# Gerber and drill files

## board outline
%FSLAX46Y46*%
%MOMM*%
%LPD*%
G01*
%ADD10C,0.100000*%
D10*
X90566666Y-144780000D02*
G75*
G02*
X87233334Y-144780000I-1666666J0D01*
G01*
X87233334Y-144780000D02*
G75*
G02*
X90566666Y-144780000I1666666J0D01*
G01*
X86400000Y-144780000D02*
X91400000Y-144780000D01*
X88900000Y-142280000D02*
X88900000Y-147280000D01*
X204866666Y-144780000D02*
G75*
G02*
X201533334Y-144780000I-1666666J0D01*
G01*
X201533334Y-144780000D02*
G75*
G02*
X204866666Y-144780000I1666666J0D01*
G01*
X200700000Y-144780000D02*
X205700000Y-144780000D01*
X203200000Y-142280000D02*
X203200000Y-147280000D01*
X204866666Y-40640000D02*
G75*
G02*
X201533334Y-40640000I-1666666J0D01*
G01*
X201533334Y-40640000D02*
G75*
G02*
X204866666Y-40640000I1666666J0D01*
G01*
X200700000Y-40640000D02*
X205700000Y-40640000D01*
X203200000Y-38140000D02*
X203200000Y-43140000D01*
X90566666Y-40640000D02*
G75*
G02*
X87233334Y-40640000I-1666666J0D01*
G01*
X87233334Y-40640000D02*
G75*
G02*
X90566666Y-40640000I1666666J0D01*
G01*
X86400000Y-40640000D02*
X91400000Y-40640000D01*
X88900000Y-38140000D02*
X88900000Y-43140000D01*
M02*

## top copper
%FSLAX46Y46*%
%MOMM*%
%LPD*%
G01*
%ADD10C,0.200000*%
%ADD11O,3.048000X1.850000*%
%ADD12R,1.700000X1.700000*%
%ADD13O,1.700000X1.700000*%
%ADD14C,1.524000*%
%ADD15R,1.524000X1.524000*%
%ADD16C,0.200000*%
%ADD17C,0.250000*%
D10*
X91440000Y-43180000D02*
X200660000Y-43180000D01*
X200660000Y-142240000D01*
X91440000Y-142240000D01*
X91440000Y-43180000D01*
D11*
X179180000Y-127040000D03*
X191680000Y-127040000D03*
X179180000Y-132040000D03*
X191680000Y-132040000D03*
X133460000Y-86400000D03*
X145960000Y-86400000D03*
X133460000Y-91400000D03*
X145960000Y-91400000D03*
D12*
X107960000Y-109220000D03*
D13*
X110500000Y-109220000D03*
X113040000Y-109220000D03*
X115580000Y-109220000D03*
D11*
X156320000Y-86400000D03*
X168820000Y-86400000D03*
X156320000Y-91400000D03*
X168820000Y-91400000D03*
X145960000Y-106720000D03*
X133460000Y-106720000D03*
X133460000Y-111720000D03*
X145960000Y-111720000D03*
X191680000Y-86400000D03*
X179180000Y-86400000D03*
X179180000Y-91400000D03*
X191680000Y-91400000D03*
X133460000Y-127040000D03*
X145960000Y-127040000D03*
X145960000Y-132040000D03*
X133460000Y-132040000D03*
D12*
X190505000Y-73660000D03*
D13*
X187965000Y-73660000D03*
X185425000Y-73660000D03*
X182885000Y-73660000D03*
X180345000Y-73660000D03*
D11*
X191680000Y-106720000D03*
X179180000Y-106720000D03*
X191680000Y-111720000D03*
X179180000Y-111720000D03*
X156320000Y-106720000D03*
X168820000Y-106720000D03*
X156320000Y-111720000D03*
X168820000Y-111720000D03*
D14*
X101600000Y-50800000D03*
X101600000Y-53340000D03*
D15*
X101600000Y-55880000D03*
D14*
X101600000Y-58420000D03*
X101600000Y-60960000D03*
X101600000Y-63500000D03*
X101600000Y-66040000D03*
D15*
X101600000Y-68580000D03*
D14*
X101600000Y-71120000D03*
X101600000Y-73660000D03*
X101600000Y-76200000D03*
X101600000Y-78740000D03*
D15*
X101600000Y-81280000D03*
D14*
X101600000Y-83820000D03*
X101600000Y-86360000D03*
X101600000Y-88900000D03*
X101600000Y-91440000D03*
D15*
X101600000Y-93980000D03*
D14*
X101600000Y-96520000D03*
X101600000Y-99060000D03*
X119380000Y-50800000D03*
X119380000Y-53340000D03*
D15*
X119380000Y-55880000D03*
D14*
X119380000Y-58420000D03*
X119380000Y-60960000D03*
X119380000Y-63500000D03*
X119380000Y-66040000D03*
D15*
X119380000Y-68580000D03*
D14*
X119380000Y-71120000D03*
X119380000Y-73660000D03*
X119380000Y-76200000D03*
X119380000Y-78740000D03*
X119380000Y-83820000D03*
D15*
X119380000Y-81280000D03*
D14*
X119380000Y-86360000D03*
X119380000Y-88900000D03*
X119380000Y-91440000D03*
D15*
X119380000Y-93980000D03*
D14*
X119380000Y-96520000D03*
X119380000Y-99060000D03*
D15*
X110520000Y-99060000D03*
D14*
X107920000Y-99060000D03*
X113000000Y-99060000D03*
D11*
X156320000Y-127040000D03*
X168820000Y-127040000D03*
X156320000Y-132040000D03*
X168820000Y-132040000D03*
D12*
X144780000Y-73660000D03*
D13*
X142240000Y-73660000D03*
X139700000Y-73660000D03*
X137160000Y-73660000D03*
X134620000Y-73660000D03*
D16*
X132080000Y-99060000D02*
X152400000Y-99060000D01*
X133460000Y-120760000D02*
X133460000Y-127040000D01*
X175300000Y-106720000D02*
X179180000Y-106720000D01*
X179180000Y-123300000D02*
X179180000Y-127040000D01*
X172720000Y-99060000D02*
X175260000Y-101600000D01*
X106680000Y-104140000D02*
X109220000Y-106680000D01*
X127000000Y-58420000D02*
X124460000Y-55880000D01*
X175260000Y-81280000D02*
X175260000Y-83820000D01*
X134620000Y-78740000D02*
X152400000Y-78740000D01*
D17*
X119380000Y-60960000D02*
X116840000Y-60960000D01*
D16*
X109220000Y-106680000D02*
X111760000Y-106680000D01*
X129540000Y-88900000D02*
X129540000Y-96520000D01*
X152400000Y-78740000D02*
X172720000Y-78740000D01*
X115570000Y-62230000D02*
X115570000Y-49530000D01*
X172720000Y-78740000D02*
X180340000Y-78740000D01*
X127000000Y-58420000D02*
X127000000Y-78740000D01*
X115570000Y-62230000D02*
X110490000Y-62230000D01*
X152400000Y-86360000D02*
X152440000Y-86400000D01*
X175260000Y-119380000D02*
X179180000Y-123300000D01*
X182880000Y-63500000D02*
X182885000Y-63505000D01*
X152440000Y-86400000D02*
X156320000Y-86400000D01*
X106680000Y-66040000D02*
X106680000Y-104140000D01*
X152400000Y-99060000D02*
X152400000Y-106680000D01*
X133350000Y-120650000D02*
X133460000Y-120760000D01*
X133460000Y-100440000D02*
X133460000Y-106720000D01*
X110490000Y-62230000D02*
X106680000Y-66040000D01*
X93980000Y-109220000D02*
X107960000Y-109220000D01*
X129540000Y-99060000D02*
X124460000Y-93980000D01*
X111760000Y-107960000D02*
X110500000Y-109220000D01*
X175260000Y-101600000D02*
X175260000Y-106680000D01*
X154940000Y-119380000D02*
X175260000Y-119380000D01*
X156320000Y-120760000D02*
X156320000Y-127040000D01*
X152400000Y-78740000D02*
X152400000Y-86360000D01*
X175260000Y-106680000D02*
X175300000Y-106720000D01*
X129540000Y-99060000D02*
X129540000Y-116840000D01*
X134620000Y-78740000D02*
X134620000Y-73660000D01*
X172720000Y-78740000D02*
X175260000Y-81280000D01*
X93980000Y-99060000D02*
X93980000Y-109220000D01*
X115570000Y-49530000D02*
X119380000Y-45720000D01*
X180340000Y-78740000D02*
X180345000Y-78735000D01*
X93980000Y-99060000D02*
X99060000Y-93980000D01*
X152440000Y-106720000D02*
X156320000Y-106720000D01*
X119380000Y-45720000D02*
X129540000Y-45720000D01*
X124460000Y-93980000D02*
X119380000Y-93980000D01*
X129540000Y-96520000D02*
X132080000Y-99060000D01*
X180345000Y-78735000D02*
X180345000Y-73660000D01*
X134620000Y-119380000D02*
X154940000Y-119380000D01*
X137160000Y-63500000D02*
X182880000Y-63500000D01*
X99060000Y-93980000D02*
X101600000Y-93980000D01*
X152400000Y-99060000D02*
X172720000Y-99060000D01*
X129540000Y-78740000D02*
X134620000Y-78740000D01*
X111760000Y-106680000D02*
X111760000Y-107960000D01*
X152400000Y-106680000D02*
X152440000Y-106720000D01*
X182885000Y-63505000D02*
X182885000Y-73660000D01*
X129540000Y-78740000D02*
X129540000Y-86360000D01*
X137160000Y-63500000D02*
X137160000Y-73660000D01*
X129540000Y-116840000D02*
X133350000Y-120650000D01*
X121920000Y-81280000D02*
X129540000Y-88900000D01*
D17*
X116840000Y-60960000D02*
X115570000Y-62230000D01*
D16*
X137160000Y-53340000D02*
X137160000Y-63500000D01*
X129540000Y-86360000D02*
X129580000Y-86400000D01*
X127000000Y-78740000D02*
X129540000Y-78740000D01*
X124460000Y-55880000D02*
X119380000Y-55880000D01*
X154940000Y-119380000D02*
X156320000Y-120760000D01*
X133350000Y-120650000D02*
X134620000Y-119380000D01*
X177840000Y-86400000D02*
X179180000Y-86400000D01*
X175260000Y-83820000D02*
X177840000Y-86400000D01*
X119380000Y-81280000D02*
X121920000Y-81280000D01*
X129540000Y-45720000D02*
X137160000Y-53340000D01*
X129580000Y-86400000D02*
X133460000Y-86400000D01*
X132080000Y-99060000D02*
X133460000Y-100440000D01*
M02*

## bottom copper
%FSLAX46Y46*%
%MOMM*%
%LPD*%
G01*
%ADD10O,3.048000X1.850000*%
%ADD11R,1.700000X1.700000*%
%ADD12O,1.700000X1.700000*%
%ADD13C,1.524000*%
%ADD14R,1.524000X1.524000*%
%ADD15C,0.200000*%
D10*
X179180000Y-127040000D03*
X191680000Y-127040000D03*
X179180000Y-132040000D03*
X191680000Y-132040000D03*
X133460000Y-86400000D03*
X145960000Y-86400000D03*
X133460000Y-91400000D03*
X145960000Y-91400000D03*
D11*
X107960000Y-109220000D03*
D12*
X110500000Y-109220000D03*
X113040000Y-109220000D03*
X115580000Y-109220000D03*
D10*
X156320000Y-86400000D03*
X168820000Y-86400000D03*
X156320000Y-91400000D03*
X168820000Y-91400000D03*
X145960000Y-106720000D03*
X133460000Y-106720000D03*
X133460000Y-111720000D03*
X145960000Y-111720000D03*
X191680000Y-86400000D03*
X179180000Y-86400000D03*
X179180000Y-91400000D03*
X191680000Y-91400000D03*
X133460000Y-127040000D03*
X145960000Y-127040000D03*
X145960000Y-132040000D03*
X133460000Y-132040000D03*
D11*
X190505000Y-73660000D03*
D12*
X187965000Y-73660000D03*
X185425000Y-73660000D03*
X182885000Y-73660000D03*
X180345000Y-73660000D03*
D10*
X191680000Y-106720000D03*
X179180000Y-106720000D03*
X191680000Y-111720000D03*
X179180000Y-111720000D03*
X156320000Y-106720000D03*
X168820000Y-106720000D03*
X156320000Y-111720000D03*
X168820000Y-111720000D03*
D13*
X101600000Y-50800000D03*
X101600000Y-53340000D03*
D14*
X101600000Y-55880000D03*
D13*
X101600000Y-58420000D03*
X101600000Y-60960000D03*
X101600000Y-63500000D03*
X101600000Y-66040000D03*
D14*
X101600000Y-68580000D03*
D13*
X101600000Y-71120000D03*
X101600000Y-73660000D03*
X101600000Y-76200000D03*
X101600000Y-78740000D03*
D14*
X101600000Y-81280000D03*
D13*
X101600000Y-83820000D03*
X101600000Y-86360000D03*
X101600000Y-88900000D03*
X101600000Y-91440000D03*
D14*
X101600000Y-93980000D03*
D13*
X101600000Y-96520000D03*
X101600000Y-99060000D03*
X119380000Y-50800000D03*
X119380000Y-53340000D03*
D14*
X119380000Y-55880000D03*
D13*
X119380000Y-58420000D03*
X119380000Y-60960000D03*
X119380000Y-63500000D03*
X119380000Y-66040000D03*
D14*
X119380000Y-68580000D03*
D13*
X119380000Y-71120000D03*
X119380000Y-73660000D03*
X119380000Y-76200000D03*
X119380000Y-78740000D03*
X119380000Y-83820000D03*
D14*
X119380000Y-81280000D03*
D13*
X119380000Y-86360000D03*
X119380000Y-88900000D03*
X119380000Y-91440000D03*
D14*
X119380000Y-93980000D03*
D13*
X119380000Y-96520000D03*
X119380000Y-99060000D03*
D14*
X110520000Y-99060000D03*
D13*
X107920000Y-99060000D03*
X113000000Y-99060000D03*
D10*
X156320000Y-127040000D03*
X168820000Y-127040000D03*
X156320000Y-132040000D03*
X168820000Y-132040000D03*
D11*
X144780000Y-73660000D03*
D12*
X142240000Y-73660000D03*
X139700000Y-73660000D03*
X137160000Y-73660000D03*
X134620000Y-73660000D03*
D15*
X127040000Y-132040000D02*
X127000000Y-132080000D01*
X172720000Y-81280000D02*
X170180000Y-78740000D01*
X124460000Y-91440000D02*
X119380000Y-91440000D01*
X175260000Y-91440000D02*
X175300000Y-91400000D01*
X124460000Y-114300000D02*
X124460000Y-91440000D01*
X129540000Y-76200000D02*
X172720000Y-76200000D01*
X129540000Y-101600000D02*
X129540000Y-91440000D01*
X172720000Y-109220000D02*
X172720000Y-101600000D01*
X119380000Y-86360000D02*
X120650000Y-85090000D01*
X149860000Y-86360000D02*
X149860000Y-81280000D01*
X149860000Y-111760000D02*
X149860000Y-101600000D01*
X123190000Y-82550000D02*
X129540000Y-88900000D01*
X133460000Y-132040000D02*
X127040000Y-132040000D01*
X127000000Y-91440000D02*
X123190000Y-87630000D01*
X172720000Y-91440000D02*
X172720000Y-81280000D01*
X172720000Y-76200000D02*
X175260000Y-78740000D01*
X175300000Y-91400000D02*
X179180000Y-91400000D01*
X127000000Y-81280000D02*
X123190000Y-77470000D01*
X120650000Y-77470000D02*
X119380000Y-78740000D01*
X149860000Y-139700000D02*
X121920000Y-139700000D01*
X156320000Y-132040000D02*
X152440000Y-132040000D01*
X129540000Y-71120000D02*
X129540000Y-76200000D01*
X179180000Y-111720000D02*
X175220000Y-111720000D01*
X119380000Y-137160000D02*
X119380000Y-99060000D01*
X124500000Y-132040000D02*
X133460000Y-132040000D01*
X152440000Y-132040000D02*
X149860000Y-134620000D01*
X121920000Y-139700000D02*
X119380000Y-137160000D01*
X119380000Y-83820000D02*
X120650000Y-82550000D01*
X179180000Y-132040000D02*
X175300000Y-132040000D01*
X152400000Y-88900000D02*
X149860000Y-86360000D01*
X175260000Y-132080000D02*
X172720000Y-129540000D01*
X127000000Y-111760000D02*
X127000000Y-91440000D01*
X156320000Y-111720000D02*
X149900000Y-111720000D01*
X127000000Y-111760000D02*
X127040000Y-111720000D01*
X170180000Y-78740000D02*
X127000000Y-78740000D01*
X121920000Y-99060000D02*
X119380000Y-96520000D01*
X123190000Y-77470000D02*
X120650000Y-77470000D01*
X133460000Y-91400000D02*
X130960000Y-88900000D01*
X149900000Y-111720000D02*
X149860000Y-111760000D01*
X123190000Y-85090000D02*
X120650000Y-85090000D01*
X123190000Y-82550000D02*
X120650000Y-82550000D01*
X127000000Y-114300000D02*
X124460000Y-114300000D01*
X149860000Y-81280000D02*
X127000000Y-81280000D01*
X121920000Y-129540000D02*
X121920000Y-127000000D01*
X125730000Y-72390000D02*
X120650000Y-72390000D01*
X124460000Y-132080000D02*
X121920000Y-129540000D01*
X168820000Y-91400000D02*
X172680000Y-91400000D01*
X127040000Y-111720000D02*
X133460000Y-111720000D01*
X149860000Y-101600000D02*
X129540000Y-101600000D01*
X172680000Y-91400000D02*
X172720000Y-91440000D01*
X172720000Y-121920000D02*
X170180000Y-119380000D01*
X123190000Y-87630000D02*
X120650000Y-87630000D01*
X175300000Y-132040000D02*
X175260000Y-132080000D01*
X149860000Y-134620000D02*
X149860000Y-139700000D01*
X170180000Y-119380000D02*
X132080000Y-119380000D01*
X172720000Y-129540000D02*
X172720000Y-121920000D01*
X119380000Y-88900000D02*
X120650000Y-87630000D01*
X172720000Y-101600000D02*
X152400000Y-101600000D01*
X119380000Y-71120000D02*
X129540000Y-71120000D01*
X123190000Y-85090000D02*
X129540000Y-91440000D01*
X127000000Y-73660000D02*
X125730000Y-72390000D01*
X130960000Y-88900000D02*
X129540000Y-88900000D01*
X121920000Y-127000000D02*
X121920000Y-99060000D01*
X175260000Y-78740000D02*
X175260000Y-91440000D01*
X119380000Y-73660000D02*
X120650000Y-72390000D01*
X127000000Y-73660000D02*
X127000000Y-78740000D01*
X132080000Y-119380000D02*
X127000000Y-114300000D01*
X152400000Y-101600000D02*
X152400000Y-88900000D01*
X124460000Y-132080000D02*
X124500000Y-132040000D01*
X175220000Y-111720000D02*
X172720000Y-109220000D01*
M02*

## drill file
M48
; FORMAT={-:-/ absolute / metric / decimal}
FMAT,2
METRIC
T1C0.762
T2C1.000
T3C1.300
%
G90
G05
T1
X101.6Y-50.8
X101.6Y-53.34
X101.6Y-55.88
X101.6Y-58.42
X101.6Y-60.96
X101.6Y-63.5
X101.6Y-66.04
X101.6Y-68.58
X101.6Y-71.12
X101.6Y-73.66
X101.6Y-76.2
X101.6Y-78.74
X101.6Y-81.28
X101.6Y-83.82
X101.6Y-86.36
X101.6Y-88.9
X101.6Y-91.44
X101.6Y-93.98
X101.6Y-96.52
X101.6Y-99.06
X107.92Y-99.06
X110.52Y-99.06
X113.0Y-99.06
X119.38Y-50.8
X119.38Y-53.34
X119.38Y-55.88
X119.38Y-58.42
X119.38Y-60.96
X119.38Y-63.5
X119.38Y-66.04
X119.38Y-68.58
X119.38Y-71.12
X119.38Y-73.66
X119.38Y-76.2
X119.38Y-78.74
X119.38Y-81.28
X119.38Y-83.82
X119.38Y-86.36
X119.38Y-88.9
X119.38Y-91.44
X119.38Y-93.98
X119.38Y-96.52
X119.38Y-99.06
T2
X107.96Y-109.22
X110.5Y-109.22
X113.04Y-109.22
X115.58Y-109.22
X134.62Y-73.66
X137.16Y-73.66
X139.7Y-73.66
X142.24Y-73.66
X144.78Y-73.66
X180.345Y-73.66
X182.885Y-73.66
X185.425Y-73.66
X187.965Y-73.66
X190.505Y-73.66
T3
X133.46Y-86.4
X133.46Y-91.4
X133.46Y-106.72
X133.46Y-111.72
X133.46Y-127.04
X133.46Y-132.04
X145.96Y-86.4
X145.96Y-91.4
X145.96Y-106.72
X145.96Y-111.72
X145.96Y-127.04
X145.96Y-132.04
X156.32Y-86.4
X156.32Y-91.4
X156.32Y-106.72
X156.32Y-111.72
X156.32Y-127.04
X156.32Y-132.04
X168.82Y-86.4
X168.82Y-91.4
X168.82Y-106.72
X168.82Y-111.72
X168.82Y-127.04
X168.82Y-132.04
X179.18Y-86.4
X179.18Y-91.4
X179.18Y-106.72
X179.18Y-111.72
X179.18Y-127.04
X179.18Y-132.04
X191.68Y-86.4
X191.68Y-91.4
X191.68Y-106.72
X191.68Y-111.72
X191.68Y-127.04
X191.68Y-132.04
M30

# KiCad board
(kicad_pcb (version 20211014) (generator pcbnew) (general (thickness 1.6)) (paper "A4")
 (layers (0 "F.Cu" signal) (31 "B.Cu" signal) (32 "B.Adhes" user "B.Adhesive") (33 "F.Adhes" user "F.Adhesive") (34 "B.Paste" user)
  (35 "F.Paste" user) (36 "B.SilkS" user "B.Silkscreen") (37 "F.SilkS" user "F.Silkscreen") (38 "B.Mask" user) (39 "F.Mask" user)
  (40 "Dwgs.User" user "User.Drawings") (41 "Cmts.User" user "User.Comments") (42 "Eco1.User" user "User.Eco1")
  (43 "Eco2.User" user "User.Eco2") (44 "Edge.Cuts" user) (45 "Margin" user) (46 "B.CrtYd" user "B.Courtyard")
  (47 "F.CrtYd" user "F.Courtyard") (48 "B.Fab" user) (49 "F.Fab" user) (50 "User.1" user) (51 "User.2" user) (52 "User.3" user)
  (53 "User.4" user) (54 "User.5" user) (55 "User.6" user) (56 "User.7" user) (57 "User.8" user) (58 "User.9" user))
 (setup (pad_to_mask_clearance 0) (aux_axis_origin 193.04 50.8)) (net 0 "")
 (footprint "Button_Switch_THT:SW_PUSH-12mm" (layer "F.Cu") (at 179.18 127.04)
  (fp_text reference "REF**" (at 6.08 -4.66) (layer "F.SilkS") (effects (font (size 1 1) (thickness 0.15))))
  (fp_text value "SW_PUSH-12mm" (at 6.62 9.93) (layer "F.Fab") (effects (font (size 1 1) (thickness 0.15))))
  (pad "1" thru_hole oval (at 0 0) (size 3.048 1.85) (drill 1.3) (layers *.Cu *.Mask))
  (pad "1" thru_hole oval (at 12.5 0) (size 3.048 1.85) (drill 1.3) (layers *.Cu *.Mask))
  (pad "2" thru_hole oval (at 0 5) (size 3.048 1.85) (drill 1.3) (layers *.Cu *.Mask))
  (pad "2" thru_hole oval (at 12.5 5) (size 3.048 1.85) (drill 1.3) (layers *.Cu *.Mask)))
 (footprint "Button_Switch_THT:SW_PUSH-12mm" (layer "F.Cu") (at 133.46 86.4)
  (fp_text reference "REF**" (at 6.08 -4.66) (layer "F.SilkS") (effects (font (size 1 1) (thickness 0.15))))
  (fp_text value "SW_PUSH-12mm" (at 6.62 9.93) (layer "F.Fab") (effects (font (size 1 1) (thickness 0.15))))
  (pad "1" thru_hole oval (at 0 0) (size 3.048 1.85) (drill 1.3) (layers *.Cu *.Mask))
  (pad "1" thru_hole oval (at 12.5 0) (size 3.048 1.85) (drill 1.3) (layers *.Cu *.Mask))
  (pad "2" thru_hole oval (at 0 5) (size 3.048 1.85) (drill 1.3) (layers *.Cu *.Mask))
  (pad "2" thru_hole oval (at 12.5 5) (size 3.048 1.85) (drill 1.3) (layers *.Cu *.Mask)))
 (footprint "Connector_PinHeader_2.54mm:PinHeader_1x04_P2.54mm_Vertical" (layer "F.Cu") (at 107.96 109.22 90)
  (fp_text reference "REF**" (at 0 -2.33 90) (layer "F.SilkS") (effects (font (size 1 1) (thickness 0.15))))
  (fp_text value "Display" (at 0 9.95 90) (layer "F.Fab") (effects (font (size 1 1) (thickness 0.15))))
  (pad "1" thru_hole rect (at 0 0 90) (size 1.7 1.7) (drill 1) (layers *.Cu *.Mask))
  (pad "2" thru_hole oval (at 0 2.54 90) (size 1.7 1.7) (drill 1) (layers *.Cu *.Mask))
  (pad "3" thru_hole oval (at 0 5.08 90) (size 1.7 1.7) (drill 1) (layers *.Cu *.Mask))
  (pad "4" thru_hole oval (at 0 7.62 90) (size 1.7 1.7) (drill 1) (layers *.Cu *.Mask)))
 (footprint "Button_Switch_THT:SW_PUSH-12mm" (layer "F.Cu") (at 156.32 86.4)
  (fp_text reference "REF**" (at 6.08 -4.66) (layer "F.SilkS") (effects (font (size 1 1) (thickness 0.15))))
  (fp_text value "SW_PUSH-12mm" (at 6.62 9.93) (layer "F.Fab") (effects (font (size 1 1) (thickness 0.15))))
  (pad "1" thru_hole oval (at 0 0) (size 3.048 1.85) (drill 1.3) (layers *.Cu *.Mask))
  (pad "1" thru_hole oval (at 12.5 0) (size 3.048 1.85) (drill 1.3) (layers *.Cu *.Mask))
  (pad "2" thru_hole oval (at 0 5) (size 3.048 1.85) (drill 1.3) (layers *.Cu *.Mask))
  (pad "2" thru_hole oval (at 12.5 5) (size 3.048 1.85) (drill 1.3) (layers *.Cu *.Mask)))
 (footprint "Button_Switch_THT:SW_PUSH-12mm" (layer "F.Cu") (at 133.46 106.72)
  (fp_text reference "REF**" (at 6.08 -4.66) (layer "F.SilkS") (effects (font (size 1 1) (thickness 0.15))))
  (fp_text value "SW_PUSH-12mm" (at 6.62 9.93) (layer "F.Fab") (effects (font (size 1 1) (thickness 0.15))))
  (pad "1" thru_hole oval (at 12.5 0) (size 3.048 1.85) (drill 1.3) (layers *.Cu *.Mask))
  (pad "1" thru_hole oval (at 0 0) (size 3.048 1.85) (drill 1.3) (layers *.Cu *.Mask))
  (pad "2" thru_hole oval (at 0 5) (size 3.048 1.85) (drill 1.3) (layers *.Cu *.Mask))
  (pad "2" thru_hole oval (at 12.5 5) (size 3.048 1.85) (drill 1.3) (layers *.Cu *.Mask)))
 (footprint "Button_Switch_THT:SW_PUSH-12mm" (layer "F.Cu") (at 179.18 86.4)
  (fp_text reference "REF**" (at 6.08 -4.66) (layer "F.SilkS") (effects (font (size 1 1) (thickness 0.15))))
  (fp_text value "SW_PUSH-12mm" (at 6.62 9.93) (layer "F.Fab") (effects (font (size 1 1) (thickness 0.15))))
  (pad "1" thru_hole oval (at 12.5 0) (size 3.048 1.85) (drill 1.3) (layers *.Cu *.Mask))
  (pad "1" thru_hole oval (at 0 0) (size 3.048 1.85) (drill 1.3) (layers *.Cu *.Mask))
  (pad "2" thru_hole oval (at 0 5) (size 3.048 1.85) (drill 1.3) (layers *.Cu *.Mask))
  (pad "2" thru_hole oval (at 12.5 5) (size 3.048 1.85) (drill 1.3) (layers *.Cu *.Mask)))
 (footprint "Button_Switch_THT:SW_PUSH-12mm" (layer "F.Cu") (at 133.46 127.04)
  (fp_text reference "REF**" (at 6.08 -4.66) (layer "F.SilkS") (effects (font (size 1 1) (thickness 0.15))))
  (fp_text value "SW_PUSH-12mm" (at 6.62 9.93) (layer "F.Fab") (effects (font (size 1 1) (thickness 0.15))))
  (pad "1" thru_hole oval (at 0 0) (size 3.048 1.85) (drill 1.3) (layers *.Cu *.Mask))
  (pad "1" thru_hole oval (at 12.5 0) (size 3.048 1.85) (drill 1.3) (layers *.Cu *.Mask))
  (pad "2" thru_hole oval (at 12.5 5) (size 3.048 1.85) (drill 1.3) (layers *.Cu *.Mask))
  (pad "2" thru_hole oval (at 0 5) (size 3.048 1.85) (drill 1.3) (layers *.Cu *.Mask)))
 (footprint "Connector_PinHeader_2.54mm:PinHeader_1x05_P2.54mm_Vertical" (layer "F.Cu") (at 190.505 73.66 -90)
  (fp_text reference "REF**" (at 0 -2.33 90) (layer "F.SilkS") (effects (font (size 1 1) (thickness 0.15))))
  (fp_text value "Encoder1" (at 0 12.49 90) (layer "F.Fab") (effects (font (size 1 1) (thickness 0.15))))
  (pad "1" thru_hole rect (at 0 0 270) (size 1.7 1.7) (drill 1) (layers *.Cu *.Mask))
  (pad "2" thru_hole oval (at 0 2.54 270) (size 1.7 1.7) (drill 1) (layers *.Cu *.Mask))
  (pad "3" thru_hole oval (at 0 5.08 270) (size 1.7 1.7) (drill 1) (layers *.Cu *.Mask))
  (pad "4" thru_hole oval (at 0 7.62 270) (size 1.7 1.7) (drill 1) (layers *.Cu *.Mask))
  (pad "5" thru_hole oval (at 0 10.16 270) (size 1.7 1.7) (drill 1) (layers *.Cu *.Mask)))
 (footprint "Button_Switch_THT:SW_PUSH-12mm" (layer "F.Cu") (at 179.18 106.72)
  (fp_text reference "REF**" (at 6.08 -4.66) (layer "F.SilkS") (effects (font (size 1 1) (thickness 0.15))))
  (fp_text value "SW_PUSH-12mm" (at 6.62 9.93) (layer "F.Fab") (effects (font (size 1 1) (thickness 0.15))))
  (pad "1" thru_hole oval (at 12.5 0) (size 3.048 1.85) (drill 1.3) (layers *.Cu *.Mask))
  (pad "1" thru_hole oval (at 0 0) (size 3.048 1.85) (drill 1.3) (layers *.Cu *.Mask))
  (pad "2" thru_hole oval (at 12.5 5) (size 3.048 1.85) (drill 1.3) (layers *.Cu *.Mask))
  (pad "2" thru_hole oval (at 0 5) (size 3.048 1.85) (drill 1.3) (layers *.Cu *.Mask)))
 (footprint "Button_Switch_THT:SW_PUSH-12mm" (layer "F.Cu") (at 156.32 106.72)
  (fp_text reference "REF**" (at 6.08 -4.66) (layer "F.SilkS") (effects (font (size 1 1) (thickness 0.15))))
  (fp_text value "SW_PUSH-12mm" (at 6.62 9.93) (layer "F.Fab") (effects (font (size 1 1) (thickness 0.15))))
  (pad "1" thru_hole oval (at 0 0) (size 3.048 1.85) (drill 1.3) (layers *.Cu *.Mask))
  (pad "1" thru_hole oval (at 12.5 0) (size 3.048 1.85) (drill 1.3) (layers *.Cu *.Mask))
  (pad "2" thru_hole oval (at 0 5) (size 3.048 1.85) (drill 1.3) (layers *.Cu *.Mask))
  (pad "2" thru_hole oval (at 12.5 5) (size 3.048 1.85) (drill 1.3) (layers *.Cu *.Mask)))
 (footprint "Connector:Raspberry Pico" (layer "F.Cu") (at 101.6 78.74)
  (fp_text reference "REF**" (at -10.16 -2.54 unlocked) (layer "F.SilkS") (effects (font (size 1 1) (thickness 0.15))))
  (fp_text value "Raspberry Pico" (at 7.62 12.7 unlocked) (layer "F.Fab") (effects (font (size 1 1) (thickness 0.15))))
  (pad "1" thru_hole circle (at 0 -27.94) (size 1.524 1.524) (drill 0.762) (layers *.Cu *.Mask))
  (pad "2" thru_hole circle (at 0 -25.4) (size 1.524 1.524) (drill 0.762) (layers *.Cu *.Mask))
  (pad "3" thru_hole rect (at 0 -22.86) (size 1.524 1.524) (drill 0.762) (layers *.Cu *.Mask))
  (pad "4" thru_hole circle (at 0 -20.32) (size 1.524 1.524) (drill 0.762) (layers *.Cu *.Mask))
  (pad "5" thru_hole circle (at 0 -17.78) (size 1.524 1.524) (drill 0.762) (layers *.Cu *.Mask))
  (pad "6" thru_hole circle (at 0 -15.24) (size 1.524 1.524) (drill 0.762) (layers *.Cu *.Mask))
  (pad "7" thru_hole circle (at 0 -12.7) (size 1.524 1.524) (drill 0.762) (layers *.Cu *.Mask))
  (pad "8" thru_hole rect (at 0 -10.16) (size 1.524 1.524) (drill 0.762) (layers *.Cu *.Mask))
  (pad "9" thru_hole circle (at 0 -7.62) (size 1.524 1.524) (drill 0.762) (layers *.Cu *.Mask))
  (pad "10" thru_hole circle (at 0 -5.08) (size 1.524 1.524) (drill 0.762) (layers *.Cu *.Mask))
  (pad "11" thru_hole circle (at 0 -2.54) (size 1.524 1.524) (drill 0.762) (layers *.Cu *.Mask))
  (pad "12" thru_hole circle (at 0 0) (size 1.524 1.524) (drill 0.762) (layers *.Cu *.Mask))
  (pad "13" thru_hole rect (at 0 2.54) (size 1.524 1.524) (drill 0.762) (layers *.Cu *.Mask))
  (pad "14" thru_hole circle (at 0 5.08) (size 1.524 1.524) (drill 0.762) (layers *.Cu *.Mask))
  (pad "15" thru_hole circle (at 0 7.62) (size 1.524 1.524) (drill 0.762) (layers *.Cu *.Mask))
  (pad "16" thru_hole circle (at 0 10.16) (size 1.524 1.524) (drill 0.762) (layers *.Cu *.Mask))
  (pad "17" thru_hole circle (at 0 12.7) (size 1.524 1.524) (drill 0.762) (layers *.Cu *.Mask))
  (pad "18" thru_hole rect (at 0 15.24) (size 1.524 1.524) (drill 0.762) (layers *.Cu *.Mask))
  (pad "19" thru_hole circle (at 0 17.78) (size 1.524 1.524) (drill 0.762) (layers *.Cu *.Mask))
  (pad "19" thru_hole circle (at 0 20.32) (size 1.524 1.524) (drill 0.762) (layers *.Cu *.Mask))
  (pad "20" thru_hole circle (at 17.78 -27.94) (size 1.524 1.524) (drill 0.762) (layers *.Cu *.Mask))
  (pad "21" thru_hole circle (at 17.78 -25.4) (size 1.524 1.524) (drill 0.762) (layers *.Cu *.Mask))
  (pad "22" thru_hole rect (at 17.78 -22.86) (size 1.524 1.524) (drill 0.762) (layers *.Cu *.Mask))
  (pad "23" thru_hole circle (at 17.78 -20.32) (size 1.524 1.524) (drill 0.762) (layers *.Cu *.Mask))
  (pad "24" thru_hole circle (at 17.78 -17.78) (size 1.524 1.524) (drill 0.762) (layers *.Cu *.Mask))
  (pad "25" thru_hole circle (at 17.78 -15.24) (size 1.524 1.524) (drill 0.762) (layers *.Cu *.Mask))
  (pad "26" thru_hole circle (at 17.78 -12.7) (size 1.524 1.524) (drill 0.762) (layers *.Cu *.Mask))
  (pad "27" thru_hole rect (at 17.78 -10.16) (size 1.524 1.524) (drill 0.762) (layers *.Cu *.Mask))
  (pad "28" thru_hole circle (at 17.78 -7.62) (size 1.524 1.524) (drill 0.762) (layers *.Cu *.Mask))
  (pad "29" thru_hole circle (at 17.78 -5.08) (size 1.524 1.524) (drill 0.762) (layers *.Cu *.Mask))
  (pad "30" thru_hole circle (at 17.78 -2.54) (size 1.524 1.524) (drill 0.762) (layers *.Cu *.Mask))
  (pad "31" thru_hole circle (at 17.78 0) (size 1.524 1.524) (drill 0.762) (layers *.Cu *.Mask))
  (pad "32" thru_hole circle (at 17.78 5.08) (size 1.524 1.524) (drill 0.762) (layers *.Cu *.Mask))
  (pad "33" thru_hole rect (at 17.78 2.54) (size 1.524 1.524) (drill 0.762) (layers *.Cu *.Mask))
  (pad "34" thru_hole circle (at 17.78 7.62) (size 1.524 1.524) (drill 0.762) (layers *.Cu *.Mask))
  (pad "35" thru_hole circle (at 17.78 10.16) (size 1.524 1.524) (drill 0.762) (layers *.Cu *.Mask))
  (pad "36" thru_hole circle (at 17.78 12.7) (size 1.524 1.524) (drill 0.762) (layers *.Cu *.Mask))
  (pad "37" thru_hole rect (at 17.78 15.24) (size 1.524 1.524) (drill 0.762) (layers *.Cu *.Mask))
  (pad "38" thru_hole circle (at 17.78 17.78) (size 1.524 1.524) (drill 0.762) (layers *.Cu *.Mask))
  (pad "38" thru_hole circle (at 17.78 20.32) (size 1.524 1.524) (drill 0.762) (layers *.Cu *.Mask))
  (pad "39" thru_hole rect (at 8.92 20.32) (size 1.524 1.524) (drill 0.762) (layers *.Cu *.Mask))
  (pad "40" thru_hole circle (at 6.32 20.32) (size 1.524 1.524) (drill 0.762) (layers *.Cu *.Mask))
  (pad "41" thru_hole circle (at 11.4 20.32) (size 1.524 1.524) (drill 0.762) (layers *.Cu *.Mask)))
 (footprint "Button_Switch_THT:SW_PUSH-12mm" (layer "F.Cu") (at 156.32 127.04)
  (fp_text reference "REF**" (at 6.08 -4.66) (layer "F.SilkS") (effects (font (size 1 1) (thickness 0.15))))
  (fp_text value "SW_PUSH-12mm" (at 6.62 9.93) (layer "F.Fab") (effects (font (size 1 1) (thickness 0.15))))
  (pad "1" thru_hole oval (at 0 0) (size 3.048 1.85) (drill 1.3) (layers *.Cu *.Mask))
  (pad "1" thru_hole oval (at 12.5 0) (size 3.048 1.85) (drill 1.3) (layers *.Cu *.Mask))
  (pad "2" thru_hole oval (at 0 5) (size 3.048 1.85) (drill 1.3) (layers *.Cu *.Mask))
  (pad "2" thru_hole oval (at 12.5 5) (size 3.048 1.85) (drill 1.3) (layers *.Cu *.Mask)))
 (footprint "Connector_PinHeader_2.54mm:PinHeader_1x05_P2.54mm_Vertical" (layer "F.Cu") (at 144.78 73.66 -90)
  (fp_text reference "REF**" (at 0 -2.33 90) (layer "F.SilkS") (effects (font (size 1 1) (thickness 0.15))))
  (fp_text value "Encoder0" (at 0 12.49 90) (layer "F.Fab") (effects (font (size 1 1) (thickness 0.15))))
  (pad "1" thru_hole rect (at 0 0 270) (size 1.7 1.7) (drill 1) (layers *.Cu *.Mask))
  (pad "2" thru_hole oval (at 0 2.54 270) (size 1.7 1.7) (drill 1) (layers *.Cu *.Mask))
  (pad "3" thru_hole oval (at 0 5.08 270) (size 1.7 1.7) (drill 1) (layers *.Cu *.Mask))
  (pad "4" thru_hole oval (at 0 7.62 270) (size 1.7 1.7) (drill 1) (layers *.Cu *.Mask))
  (pad "5" thru_hole oval (at 0 10.16 270) (size 1.7 1.7) (drill 1) (layers *.Cu *.Mask)))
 (gr_rect (start 91.44 43.18) (end 200.66 142.24) (layer "F.Cu") (width 0.2) (fill none))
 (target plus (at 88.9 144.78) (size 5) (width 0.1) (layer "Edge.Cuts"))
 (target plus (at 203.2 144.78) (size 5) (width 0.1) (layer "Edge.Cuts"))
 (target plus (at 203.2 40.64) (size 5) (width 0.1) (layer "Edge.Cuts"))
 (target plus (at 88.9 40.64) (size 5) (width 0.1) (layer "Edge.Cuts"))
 (segment (start 132.08 99.06) (end 152.4 99.06) (width 0.2) (layer "F.Cu") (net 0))
 (segment (start 133.46 120.76) (end 133.46 127.04) (width 0.2) (layer "F.Cu") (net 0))
 (segment (start 175.3 106.72) (end 179.18 106.72) (width 0.2) (layer "F.Cu") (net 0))
 (segment (start 179.18 123.3) (end 179.18 127.04) (width 0.2) (layer "F.Cu") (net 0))
 (segment (start 172.72 99.06) (end 175.26 101.6) (width 0.2) (layer "F.Cu") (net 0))
 (segment (start 106.68 104.14) (end 109.22 106.68) (width 0.2) (layer "F.Cu") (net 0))
 (segment (start 127 58.42) (end 124.46 55.88) (width 0.2) (layer "F.Cu") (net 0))
 (segment (start 175.26 81.28) (end 175.26 83.82) (width 0.2) (layer "F.Cu") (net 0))
 (segment (start 134.62 78.74) (end 152.4 78.74) (width 0.2) (layer "F.Cu") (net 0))
 (segment (start 119.38 60.96) (end 116.84 60.96) (width 0.25) (layer "F.Cu") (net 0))
 (segment (start 109.22 106.68) (end 111.76 106.68) (width 0.2) (layer "F.Cu") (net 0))
 (segment (start 129.54 88.9) (end 129.54 96.52) (width 0.2) (layer "F.Cu") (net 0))
 (segment (start 152.4 78.74) (end 172.72 78.74) (width 0.2) (layer "F.Cu") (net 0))
 (segment (start 115.57 62.23) (end 115.57 49.53) (width 0.2) (layer "F.Cu") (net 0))
 (segment (start 172.72 78.74) (end 180.34 78.74) (width 0.2) (layer "F.Cu") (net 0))
 (segment (start 127 58.42) (end 127 78.74) (width 0.2) (layer "F.Cu") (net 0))
 (segment (start 115.57 62.23) (end 110.49 62.23) (width 0.2) (layer "F.Cu") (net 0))
 (segment (start 152.4 86.36) (end 152.44 86.4) (width 0.2) (layer "F.Cu") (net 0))
 (segment (start 175.26 119.38) (end 179.18 123.3) (width 0.2) (layer "F.Cu") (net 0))
 (segment (start 182.88 63.5) (end 182.885 63.505) (width 0.2) (layer "F.Cu") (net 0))
 (segment (start 152.44 86.4) (end 156.32 86.4) (width 0.2) (layer "F.Cu") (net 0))
 (segment (start 106.68 66.04) (end 106.68 104.14) (width 0.2) (layer "F.Cu") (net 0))
 (segment (start 152.4 99.06) (end 152.4 106.68) (width 0.2) (layer "F.Cu") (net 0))
 (segment (start 133.35 120.65) (end 133.46 120.76) (width 0.2) (layer "F.Cu") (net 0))
 (segment (start 133.46 100.44) (end 133.46 106.72) (width 0.2) (layer "F.Cu") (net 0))
 (segment (start 110.49 62.23) (end 106.68 66.04) (width 0.2) (layer "F.Cu") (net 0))
 (segment (start 93.98 109.22) (end 107.96 109.22) (width 0.2) (layer "F.Cu") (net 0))
 (segment (start 129.54 99.06) (end 124.46 93.98) (width 0.2) (layer "F.Cu") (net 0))
 (segment (start 111.76 107.96) (end 110.5 109.22) (width 0.2) (layer "F.Cu") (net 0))
 (segment (start 175.26 101.6) (end 175.26 106.68) (width 0.2) (layer "F.Cu") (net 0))
 (segment (start 154.94 119.38) (end 175.26 119.38) (width 0.2) (layer "F.Cu") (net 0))
 (segment (start 156.32 120.76) (end 156.32 127.04) (width 0.2) (layer "F.Cu") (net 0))
 (segment (start 152.4 78.74) (end 152.4 86.36) (width 0.2) (layer "F.Cu") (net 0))
 (segment (start 175.26 106.68) (end 175.3 106.72) (width 0.2) (layer "F.Cu") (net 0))
 (segment (start 129.54 99.06) (end 129.54 116.84) (width 0.2) (layer "F.Cu") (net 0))
 (segment (start 134.62 78.74) (end 134.62 73.66) (width 0.2) (layer "F.Cu") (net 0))
 (segment (start 172.72 78.74) (end 175.26 81.28) (width 0.2) (layer "F.Cu") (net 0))
 (segment (start 93.98 99.06) (end 93.98 109.22) (width 0.2) (layer "F.Cu") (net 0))
 (segment (start 115.57 49.53) (end 119.38 45.72) (width 0.2) (layer "F.Cu") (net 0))
 (segment (start 180.34 78.74) (end 180.345 78.735) (width 0.2) (layer "F.Cu") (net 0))
 (segment (start 93.98 99.06) (end 99.06 93.98) (width 0.2) (layer "F.Cu") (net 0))
 (segment (start 152.44 106.72) (end 156.32 106.72) (width 0.2) (layer "F.Cu") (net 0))
 (segment (start 119.38 45.72) (end 129.54 45.72) (width 0.2) (layer "F.Cu") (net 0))
 (segment (start 124.46 93.98) (end 119.38 93.98) (width 0.2) (layer "F.Cu") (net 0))
 (segment (start 129.54 96.52) (end 132.08 99.06) (width 0.2) (layer "F.Cu") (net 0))
 (segment (start 180.345 78.735) (end 180.345 73.66) (width 0.2) (layer "F.Cu") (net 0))
 (segment (start 134.62 119.38) (end 154.94 119.38) (width 0.2) (layer "F.Cu") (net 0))
 (segment (start 137.16 63.5) (end 182.88 63.5) (width 0.2) (layer "F.Cu") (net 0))
 (segment (start 99.06 93.98) (end 101.6 93.98) (width 0.2) (layer "F.Cu") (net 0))
 (segment (start 152.4 99.06) (end 172.72 99.06) (width 0.2) (layer "F.Cu") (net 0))
 (segment (start 129.54 78.74) (end 134.62 78.74) (width 0.2) (layer "F.Cu") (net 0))
 (segment (start 111.76 106.68) (end 111.76 107.96) (width 0.2) (layer "F.Cu") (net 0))
 (segment (start 152.4 106.68) (end 152.44 106.72) (width 0.2) (layer "F.Cu") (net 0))
 (segment (start 182.885 63.505) (end 182.885 73.66) (width 0.2) (layer "F.Cu") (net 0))
 (segment (start 129.54 78.74) (end 129.54 86.36) (width 0.2) (layer "F.Cu") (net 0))
 (segment (start 137.16 63.5) (end 137.16 73.66) (width 0.2) (layer "F.Cu") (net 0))
 (segment (start 129.54 116.84) (end 133.35 120.65) (width 0.2) (layer "F.Cu") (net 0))
 (segment (start 121.92 81.28) (end 129.54 88.9) (width 0.2) (layer "F.Cu") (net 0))
 (segment (start 116.84 60.96) (end 115.57 62.23) (width 0.25) (layer "F.Cu") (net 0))
 (segment (start 137.16 53.34) (end 137.16 63.5) (width 0.2) (layer "F.Cu") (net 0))
 (segment (start 129.54 86.36) (end 129.58 86.4) (width 0.2) (layer "F.Cu") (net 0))
 (segment (start 127 78.74) (end 129.54 78.74) (width 0.2) (layer "F.Cu") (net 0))
 (segment (start 124.46 55.88) (end 119.38 55.88) (width 0.2) (layer "F.Cu") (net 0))
 (segment (start 154.94 119.38) (end 156.32 120.76) (width 0.2) (layer "F.Cu") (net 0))
 (segment (start 133.35 120.65) (end 134.62 119.38) (width 0.2) (layer "F.Cu") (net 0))
 (segment (start 177.84 86.4) (end 179.18 86.4) (width 0.2) (layer "F.Cu") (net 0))
 (segment (start 175.26 83.82) (end 177.84 86.4) (width 0.2) (layer "F.Cu") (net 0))
 (segment (start 119.38 81.28) (end 121.92 81.28) (width 0.2) (layer "F.Cu") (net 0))
 (segment (start 129.54 45.72) (end 137.16 53.34) (width 0.2) (layer "F.Cu") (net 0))
 (segment (start 129.58 86.4) (end 133.46 86.4) (width 0.2) (layer "F.Cu") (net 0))
 (segment (start 132.08 99.06) (end 133.46 100.44) (width 0.2) (layer "F.Cu") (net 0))
 (segment (start 127.04 132.04) (end 127 132.08) (width 0.2) (layer "B.Cu") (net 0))
 (segment (start 172.72 81.28) (end 170.18 78.74) (width 0.2) (layer "B.Cu") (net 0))
 (segment (start 124.46 91.44) (end 119.38 91.44) (width 0.2) (layer "B.Cu") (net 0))
 (segment (start 175.26 91.44) (end 175.3 91.4) (width 0.2) (layer "B.Cu") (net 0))
 (segment (start 124.46 114.3) (end 124.46 91.44) (width 0.2) (layer "B.Cu") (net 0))
 (segment (start 129.54 76.2) (end 172.72 76.2) (width 0.2) (layer "B.Cu") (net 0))
 (segment (start 129.54 101.6) (end 129.54 91.44) (width 0.2) (layer "B.Cu") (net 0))
 (segment (start 172.72 109.22) (end 172.72 101.6) (width 0.2) (layer "B.Cu") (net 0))
 (segment (start 119.38 86.36) (end 120.65 85.09) (width 0.2) (layer "B.Cu") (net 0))
 (segment (start 149.86 86.36) (end 149.86 81.28) (width 0.2) (layer "B.Cu") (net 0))
 (segment (start 149.86 111.76) (end 149.86 101.6) (width 0.2) (layer "B.Cu") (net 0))
 (segment (start 123.19 82.55) (end 129.54 88.9) (width 0.2) (layer "B.Cu") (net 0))
 (segment (start 133.46 132.04) (end 127.04 132.04) (width 0.2) (layer "B.Cu") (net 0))
 (segment (start 127 91.44) (end 123.19 87.63) (width 0.2) (layer "B.Cu") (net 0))
 (segment (start 172.72 91.44) (end 172.72 81.28) (width 0.2) (layer "B.Cu") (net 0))
 (segment (start 172.72 76.2) (end 175.26 78.74) (width 0.2) (layer "B.Cu") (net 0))
 (segment (start 175.3 91.4) (end 179.18 91.4) (width 0.2) (layer "B.Cu") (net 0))
 (segment (start 127 81.28) (end 123.19 77.47) (width 0.2) (layer "B.Cu") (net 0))
 (segment (start 120.65 77.47) (end 119.38 78.74) (width 0.2) (layer "B.Cu") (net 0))
 (segment (start 149.86 139.7) (end 121.92 139.7) (width 0.2) (layer "B.Cu") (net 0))
 (segment (start 156.32 132.04) (end 152.44 132.04) (width 0.2) (layer "B.Cu") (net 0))
 (segment (start 129.54 71.12) (end 129.54 76.2) (width 0.2) (layer "B.Cu") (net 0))
 (segment (start 179.18 111.72) (end 175.22 111.72) (width 0.2) (layer "B.Cu") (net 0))
 (segment (start 119.38 137.16) (end 119.38 99.06) (width 0.2) (layer "B.Cu") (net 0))
 (segment (start 124.5 132.04) (end 133.46 132.04) (width 0.2) (layer "B.Cu") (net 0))
 (segment (start 152.44 132.04) (end 149.86 134.62) (width 0.2) (layer "B.Cu") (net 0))
 (segment (start 121.92 139.7) (end 119.38 137.16) (width 0.2) (layer "B.Cu") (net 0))
 (segment (start 119.38 83.82) (end 120.65 82.55) (width 0.2) (layer "B.Cu") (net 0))
 (segment (start 179.18 132.04) (end 175.3 132.04) (width 0.2) (layer "B.Cu") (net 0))
 (segment (start 152.4 88.9) (end 149.86 86.36) (width 0.2) (layer "B.Cu") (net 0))
 (segment (start 175.26 132.08) (end 172.72 129.54) (width 0.2) (layer "B.Cu") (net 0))
 (segment (start 127 111.76) (end 127 91.44) (width 0.2) (layer "B.Cu") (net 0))
 (segment (start 156.32 111.72) (end 149.9 111.72) (width 0.2) (layer "B.Cu") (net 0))
 (segment (start 127 111.76) (end 127.04 111.72) (width 0.2) (layer "B.Cu") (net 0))
 (segment (start 170.18 78.74) (end 127 78.74) (width 0.2) (layer "B.Cu") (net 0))
 (segment (start 121.92 99.06) (end 119.38 96.52) (width 0.2) (layer "B.Cu") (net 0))
 (segment (start 123.19 77.47) (end 120.65 77.47) (width 0.2) (layer "B.Cu") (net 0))
 (segment (start 133.46 91.4) (end 130.96 88.9) (width 0.2) (layer "B.Cu") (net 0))
 (segment (start 149.9 111.72) (end 149.86 111.76) (width 0.2) (layer "B.Cu") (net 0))
 (segment (start 123.19 85.09) (end 120.65 85.09) (width 0.2) (layer "B.Cu") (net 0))
 (segment (start 123.19 82.55) (end 120.65 82.55) (width 0.2) (layer "B.Cu") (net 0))
 (segment (start 127 114.3) (end 124.46 114.3) (width 0.2) (layer "B.Cu") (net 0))
 (segment (start 149.86 81.28) (end 127 81.28) (width 0.2) (layer "B.Cu") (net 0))
 (segment (start 121.92 129.54) (end 121.92 127) (width 0.2) (layer "B.Cu") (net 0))
 (segment (start 125.73 72.39) (end 120.65 72.39) (width 0.2) (layer "B.Cu") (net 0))
 (segment (start 124.46 132.08) (end 121.92 129.54) (width 0.2) (layer "B.Cu") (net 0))
 (segment (start 168.82 91.4) (end 172.68 91.4) (width 0.2) (layer "B.Cu") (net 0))
 (segment (start 127.04 111.72) (end 133.46 111.72) (width 0.2) (layer "B.Cu") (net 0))
 (segment (start 149.86 101.6) (end 129.54 101.6) (width 0.2) (layer "B.Cu") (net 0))
 (segment (start 172.68 91.4) (end 172.72 91.44) (width 0.2) (layer "B.Cu") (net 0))
 (segment (start 172.72 121.92) (end 170.18 119.38) (width 0.2) (layer "B.Cu") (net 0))
 (segment (start 123.19 87.63) (end 120.65 87.63) (width 0.2) (layer "B.Cu") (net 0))
 (segment (start 175.3 132.04) (end 175.26 132.08) (width 0.2) (layer "B.Cu") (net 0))
 (segment (start 149.86 134.62) (end 149.86 139.7) (width 0.2) (layer "B.Cu") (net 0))
 (segment (start 170.18 119.38) (end 132.08 119.38) (width 0.2) (layer "B.Cu") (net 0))
 (segment (start 172.72 129.54) (end 172.72 121.92) (width 0.2) (layer "B.Cu") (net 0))
 (segment (start 119.38 88.9) (end 120.65 87.63) (width 0.2) (layer "B.Cu") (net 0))
 (segment (start 172.72 101.6) (end 152.4 101.6) (width 0.2) (layer "B.Cu") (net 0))
 (segment (start 119.38 71.12) (end 129.54 71.12) (width 0.2) (layer "B.Cu") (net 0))
 (segment (start 123.19 85.09) (end 129.54 91.44) (width 0.2) (layer "B.Cu") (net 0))
 (segment (start 127 73.66) (end 125.73 72.39) (width 0.2) (layer "B.Cu") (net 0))
 (segment (start 130.96 88.9) (end 129.54 88.9) (width 0.2) (layer "B.Cu") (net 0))
 (segment (start 121.92 127) (end 121.92 99.06) (width 0.2) (layer "B.Cu") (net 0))
 (segment (start 175.26 78.74) (end 175.26 91.44) (width 0.2) (layer "B.Cu") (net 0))
 (segment (start 119.38 73.66) (end 120.65 72.39) (width 0.2) (layer "B.Cu") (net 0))
 (segment (start 127 73.66) (end 127 78.74) (width 0.2) (layer "B.Cu") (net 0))
 (segment (start 132.08 119.38) (end 127 114.3) (width 0.2) (layer "B.Cu") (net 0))
 (segment (start 152.4 101.6) (end 152.4 88.9) (width 0.2) (layer "B.Cu") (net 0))
 (segment (start 124.46 132.08) (end 124.5 132.04) (width 0.2) (layer "B.Cu") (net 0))
 (segment (start 175.22 111.72) (end 172.72 109.22) (width 0.2) (layer "B.Cu") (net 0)))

